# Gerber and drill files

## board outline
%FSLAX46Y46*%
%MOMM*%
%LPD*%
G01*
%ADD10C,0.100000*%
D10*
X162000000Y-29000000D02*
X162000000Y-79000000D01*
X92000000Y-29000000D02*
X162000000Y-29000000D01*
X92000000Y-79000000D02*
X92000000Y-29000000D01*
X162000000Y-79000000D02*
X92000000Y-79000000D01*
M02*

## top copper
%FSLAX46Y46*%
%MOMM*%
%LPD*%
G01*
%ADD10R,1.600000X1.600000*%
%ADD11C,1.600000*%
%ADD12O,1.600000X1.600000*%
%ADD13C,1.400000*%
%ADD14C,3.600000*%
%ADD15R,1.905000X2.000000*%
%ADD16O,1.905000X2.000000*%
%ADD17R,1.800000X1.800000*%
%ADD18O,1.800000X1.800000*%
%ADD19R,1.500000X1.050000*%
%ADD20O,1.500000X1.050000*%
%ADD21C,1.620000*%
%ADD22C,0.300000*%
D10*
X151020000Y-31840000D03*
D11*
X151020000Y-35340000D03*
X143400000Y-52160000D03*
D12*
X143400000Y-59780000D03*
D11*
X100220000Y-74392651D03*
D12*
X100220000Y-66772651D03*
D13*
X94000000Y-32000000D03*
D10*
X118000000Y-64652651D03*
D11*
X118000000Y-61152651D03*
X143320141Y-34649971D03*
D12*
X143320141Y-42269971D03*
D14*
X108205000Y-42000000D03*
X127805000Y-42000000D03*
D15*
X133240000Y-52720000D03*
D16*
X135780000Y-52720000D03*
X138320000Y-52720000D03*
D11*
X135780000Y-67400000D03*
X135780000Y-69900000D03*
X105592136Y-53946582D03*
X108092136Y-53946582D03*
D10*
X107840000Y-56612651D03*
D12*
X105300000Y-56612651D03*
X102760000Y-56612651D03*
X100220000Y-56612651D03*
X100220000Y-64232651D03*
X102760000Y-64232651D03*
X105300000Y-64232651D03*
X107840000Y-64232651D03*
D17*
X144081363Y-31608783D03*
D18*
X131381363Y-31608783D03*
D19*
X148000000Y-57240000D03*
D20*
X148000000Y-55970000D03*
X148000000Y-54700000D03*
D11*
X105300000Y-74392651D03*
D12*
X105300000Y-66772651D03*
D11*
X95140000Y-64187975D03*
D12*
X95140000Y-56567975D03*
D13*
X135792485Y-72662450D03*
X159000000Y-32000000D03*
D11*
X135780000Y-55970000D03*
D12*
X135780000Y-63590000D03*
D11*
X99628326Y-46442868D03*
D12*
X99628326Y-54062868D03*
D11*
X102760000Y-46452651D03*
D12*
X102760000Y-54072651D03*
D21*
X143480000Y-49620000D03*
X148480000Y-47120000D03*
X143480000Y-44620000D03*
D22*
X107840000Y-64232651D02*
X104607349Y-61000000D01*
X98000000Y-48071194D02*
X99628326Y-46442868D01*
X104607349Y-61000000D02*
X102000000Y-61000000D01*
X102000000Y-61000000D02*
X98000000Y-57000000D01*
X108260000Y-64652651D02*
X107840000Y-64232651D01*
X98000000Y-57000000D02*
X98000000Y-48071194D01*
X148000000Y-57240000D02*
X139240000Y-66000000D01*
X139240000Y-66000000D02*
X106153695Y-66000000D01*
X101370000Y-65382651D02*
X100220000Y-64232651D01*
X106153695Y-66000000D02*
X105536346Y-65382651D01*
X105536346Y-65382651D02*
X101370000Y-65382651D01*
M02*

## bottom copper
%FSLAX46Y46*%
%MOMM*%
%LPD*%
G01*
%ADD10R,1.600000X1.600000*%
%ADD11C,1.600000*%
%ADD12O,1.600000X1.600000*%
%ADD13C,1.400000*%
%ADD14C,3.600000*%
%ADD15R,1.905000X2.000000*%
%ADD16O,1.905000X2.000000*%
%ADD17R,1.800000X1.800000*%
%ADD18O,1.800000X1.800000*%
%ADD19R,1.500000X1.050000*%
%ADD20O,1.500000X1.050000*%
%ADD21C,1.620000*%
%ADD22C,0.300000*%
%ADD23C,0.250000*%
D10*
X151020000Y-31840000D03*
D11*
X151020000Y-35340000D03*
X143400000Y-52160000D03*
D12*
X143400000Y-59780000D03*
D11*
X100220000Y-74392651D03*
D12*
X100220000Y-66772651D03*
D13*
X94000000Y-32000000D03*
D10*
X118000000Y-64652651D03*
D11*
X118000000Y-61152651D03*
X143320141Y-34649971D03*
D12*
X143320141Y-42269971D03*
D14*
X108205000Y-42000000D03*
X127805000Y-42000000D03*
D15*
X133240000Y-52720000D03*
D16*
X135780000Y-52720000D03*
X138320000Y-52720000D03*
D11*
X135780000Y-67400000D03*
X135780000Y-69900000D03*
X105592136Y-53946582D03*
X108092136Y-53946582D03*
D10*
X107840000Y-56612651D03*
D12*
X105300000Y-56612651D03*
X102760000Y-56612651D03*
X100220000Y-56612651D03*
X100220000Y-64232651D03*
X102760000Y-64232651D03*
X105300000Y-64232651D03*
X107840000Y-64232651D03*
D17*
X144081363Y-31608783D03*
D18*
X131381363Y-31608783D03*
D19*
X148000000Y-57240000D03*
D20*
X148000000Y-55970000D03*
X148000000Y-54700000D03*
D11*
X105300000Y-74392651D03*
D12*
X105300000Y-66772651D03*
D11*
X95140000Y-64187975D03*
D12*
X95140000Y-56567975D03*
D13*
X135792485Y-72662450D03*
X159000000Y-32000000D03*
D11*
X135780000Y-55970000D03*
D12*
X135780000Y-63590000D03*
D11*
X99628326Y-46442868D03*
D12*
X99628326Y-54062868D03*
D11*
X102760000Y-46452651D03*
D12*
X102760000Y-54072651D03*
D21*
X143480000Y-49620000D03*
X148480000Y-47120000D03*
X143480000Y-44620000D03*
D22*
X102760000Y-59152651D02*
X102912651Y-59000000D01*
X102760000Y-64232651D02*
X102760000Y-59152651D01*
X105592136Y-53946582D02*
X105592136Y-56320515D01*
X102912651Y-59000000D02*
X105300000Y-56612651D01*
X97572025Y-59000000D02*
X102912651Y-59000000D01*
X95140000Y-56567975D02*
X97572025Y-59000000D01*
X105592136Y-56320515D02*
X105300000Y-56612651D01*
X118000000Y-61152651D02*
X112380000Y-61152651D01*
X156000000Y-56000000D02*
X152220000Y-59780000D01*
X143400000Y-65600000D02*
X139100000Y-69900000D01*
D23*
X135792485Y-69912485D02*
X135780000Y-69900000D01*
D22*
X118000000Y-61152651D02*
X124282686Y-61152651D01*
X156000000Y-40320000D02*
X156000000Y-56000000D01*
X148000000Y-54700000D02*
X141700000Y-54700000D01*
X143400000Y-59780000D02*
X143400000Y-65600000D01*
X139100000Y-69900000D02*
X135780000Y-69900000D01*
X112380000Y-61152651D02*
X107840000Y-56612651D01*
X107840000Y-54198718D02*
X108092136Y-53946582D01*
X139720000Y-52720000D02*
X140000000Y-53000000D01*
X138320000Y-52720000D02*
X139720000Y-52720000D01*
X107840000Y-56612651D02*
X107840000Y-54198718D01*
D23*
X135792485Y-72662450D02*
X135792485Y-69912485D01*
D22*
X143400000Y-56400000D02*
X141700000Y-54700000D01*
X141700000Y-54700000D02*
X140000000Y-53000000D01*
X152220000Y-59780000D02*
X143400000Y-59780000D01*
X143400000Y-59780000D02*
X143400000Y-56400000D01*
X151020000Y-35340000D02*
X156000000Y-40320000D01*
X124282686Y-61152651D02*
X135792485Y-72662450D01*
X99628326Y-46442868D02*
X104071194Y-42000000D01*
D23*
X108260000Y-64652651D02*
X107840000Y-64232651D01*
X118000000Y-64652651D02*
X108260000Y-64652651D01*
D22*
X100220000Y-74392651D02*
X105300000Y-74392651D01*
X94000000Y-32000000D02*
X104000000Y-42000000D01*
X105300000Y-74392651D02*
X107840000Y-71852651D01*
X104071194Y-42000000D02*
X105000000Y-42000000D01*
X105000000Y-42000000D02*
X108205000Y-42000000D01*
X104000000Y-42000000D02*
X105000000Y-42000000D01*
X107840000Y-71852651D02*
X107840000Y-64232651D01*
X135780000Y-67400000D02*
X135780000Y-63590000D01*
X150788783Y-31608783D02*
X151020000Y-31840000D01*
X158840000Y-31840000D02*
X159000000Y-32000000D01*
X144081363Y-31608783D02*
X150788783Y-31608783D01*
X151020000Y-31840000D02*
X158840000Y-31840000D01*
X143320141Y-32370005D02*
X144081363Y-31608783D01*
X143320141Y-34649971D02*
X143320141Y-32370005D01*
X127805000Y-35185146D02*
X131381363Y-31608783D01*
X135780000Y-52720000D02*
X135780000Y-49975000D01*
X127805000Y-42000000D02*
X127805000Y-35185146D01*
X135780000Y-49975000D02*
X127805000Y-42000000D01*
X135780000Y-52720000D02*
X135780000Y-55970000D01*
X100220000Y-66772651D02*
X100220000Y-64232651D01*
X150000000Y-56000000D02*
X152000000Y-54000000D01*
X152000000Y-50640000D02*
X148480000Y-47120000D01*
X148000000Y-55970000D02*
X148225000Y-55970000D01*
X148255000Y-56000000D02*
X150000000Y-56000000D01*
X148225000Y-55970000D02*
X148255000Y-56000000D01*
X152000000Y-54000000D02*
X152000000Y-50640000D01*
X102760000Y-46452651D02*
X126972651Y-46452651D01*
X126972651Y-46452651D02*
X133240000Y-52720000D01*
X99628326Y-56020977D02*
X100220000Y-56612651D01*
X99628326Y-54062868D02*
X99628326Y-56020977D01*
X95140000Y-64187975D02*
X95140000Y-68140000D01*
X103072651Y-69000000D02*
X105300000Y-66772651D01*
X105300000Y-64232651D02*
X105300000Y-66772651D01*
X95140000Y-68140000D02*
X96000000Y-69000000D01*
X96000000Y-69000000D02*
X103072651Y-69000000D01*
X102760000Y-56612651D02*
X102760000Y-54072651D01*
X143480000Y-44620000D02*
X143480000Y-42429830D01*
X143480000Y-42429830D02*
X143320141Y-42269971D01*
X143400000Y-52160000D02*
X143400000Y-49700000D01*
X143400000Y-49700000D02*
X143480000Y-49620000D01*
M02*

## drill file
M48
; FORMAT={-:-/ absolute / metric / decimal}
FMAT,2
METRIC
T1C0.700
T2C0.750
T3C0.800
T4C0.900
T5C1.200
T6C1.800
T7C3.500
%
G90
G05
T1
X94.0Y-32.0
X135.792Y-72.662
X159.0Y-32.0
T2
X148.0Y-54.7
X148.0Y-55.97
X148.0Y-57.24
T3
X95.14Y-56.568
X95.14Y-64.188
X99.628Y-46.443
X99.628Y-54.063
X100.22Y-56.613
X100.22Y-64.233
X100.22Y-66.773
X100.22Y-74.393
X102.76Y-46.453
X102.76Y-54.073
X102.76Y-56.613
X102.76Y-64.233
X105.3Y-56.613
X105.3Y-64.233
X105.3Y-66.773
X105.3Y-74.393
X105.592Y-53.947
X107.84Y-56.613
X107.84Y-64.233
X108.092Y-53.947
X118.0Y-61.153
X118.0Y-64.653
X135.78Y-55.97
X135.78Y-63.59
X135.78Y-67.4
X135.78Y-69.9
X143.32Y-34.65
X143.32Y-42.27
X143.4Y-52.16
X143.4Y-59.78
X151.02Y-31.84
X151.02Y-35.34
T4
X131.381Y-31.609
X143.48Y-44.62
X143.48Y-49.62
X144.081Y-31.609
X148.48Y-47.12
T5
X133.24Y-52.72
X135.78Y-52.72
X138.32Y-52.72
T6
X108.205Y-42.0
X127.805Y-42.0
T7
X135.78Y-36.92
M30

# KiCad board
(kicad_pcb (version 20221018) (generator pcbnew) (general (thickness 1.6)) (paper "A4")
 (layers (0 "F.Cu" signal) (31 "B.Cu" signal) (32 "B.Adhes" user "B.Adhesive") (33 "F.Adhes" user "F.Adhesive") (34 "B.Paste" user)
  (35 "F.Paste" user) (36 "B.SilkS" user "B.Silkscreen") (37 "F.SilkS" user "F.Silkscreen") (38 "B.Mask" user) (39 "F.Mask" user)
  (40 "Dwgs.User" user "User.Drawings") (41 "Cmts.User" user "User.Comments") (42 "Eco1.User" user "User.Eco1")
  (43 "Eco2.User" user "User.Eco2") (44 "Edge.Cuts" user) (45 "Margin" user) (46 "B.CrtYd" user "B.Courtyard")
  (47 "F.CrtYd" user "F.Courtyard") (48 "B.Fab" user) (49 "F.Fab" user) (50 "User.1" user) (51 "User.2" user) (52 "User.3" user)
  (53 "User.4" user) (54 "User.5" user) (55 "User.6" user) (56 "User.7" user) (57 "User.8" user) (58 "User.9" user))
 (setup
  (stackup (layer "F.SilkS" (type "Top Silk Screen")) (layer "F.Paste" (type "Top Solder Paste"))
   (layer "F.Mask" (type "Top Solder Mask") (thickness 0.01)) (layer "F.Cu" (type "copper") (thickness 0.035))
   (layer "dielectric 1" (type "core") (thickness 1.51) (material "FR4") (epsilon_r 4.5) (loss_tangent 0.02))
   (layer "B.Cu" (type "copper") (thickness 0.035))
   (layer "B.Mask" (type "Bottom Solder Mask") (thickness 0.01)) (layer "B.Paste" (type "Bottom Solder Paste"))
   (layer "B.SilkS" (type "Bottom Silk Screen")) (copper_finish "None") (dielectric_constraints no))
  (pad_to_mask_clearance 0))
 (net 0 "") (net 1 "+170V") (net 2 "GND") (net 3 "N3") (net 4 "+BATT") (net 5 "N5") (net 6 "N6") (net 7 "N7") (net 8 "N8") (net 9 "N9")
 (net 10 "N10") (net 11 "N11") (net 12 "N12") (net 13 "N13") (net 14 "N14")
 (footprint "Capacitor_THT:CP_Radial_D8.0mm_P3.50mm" (layer "F.Cu") (at 151.02 31.84 -90)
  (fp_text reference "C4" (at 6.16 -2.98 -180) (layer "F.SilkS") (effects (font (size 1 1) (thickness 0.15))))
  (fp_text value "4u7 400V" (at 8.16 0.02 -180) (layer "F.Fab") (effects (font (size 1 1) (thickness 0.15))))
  (pad "1" thru_hole rect (at 0 0 270) (size 1.6 1.6) (drill 0.8) (layers "*.Cu" "*.Mask") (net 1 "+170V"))
  (pad "2" thru_hole circle (at 3.5 0 270) (size 1.6 1.6) (drill 0.8) (layers "*.Cu" "*.Mask") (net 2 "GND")))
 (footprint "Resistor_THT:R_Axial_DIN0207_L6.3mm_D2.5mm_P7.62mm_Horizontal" (layer "F.Cu") (at 143.4 52.16 -90)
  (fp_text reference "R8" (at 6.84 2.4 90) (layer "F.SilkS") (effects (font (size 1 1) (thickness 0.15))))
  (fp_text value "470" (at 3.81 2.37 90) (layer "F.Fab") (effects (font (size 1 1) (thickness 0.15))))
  (pad "1" thru_hole circle (at 0 0 270) (size 1.6 1.6) (drill 0.8) (layers "*.Cu" "*.Mask") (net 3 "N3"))
  (pad "2" thru_hole oval (at 7.62 0 270) (size 1.6 1.6) (drill 0.8) (layers "*.Cu" "*.Mask") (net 2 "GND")))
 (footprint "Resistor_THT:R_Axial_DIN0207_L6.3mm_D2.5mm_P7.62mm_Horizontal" (layer "F.Cu") (at 100.22 74.392651 90)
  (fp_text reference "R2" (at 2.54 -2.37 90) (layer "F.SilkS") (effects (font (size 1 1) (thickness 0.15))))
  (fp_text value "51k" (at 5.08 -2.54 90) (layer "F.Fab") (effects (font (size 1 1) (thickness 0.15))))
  (pad "1" thru_hole circle (at 0 0 90) (size 1.6 1.6) (drill 0.8) (layers "*.Cu" "*.Mask") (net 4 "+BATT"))
  (pad "2" thru_hole oval (at 7.62 0 90) (size 1.6 1.6) (drill 0.8) (layers "*.Cu" "*.Mask") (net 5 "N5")))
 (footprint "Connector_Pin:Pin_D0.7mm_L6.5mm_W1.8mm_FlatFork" (layer "F.Cu") (at 94 32)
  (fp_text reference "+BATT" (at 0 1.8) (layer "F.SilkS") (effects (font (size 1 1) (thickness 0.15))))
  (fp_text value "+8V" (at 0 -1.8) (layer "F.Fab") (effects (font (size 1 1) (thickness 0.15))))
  (pad "1" thru_hole circle (at 0 0) (size 1.4 1.4) (drill 0.7) (layers "*.Cu" "*.Mask") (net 4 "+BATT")))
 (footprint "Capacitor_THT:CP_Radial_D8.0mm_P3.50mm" (layer "F.Cu") (at 118 64.652651 90)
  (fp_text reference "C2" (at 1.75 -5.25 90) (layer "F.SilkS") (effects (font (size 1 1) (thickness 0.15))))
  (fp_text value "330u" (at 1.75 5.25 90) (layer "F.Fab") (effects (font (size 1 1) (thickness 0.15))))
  (pad "1" thru_hole rect (at 0 0 90) (size 1.6 1.6) (drill 0.8) (layers "*.Cu" "*.Mask") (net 4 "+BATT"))
  (pad "2" thru_hole circle (at 3.5 0 90) (size 1.6 1.6) (drill 0.8) (layers "*.Cu" "*.Mask") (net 2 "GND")))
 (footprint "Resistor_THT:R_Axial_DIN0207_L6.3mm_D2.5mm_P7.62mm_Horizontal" (layer "F.Cu") (at 143.320141 34.649971 -90)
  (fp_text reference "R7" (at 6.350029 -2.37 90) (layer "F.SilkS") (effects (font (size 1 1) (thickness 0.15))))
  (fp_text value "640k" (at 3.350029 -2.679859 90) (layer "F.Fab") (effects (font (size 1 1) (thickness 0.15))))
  (pad "1" thru_hole circle (at 0 0 270) (size 1.6 1.6) (drill 0.8) (layers "*.Cu" "*.Mask") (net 1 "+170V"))
  (pad "2" thru_hole oval (at 7.62 0 270) (size 1.6 1.6) (drill 0.8) (layers "*.Cu" "*.Mask") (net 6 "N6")))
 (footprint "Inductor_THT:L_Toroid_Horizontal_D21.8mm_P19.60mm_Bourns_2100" (layer "F.Cu") (at 108.205 42)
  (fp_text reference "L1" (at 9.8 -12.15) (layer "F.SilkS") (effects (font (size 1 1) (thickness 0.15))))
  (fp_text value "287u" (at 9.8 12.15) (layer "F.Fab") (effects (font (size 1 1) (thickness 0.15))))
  (pad "1" thru_hole circle (at 0 0) (size 3.6 3.6) (drill 1.8) (layers "*.Cu" "*.Mask") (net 4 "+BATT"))
  (pad "2" thru_hole circle (at 19.6 0) (size 3.6 3.6) (drill 1.8) (layers "*.Cu" "*.Mask") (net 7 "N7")))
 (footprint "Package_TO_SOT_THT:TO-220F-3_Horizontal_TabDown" (layer "F.Cu") (at 133.24 52.72)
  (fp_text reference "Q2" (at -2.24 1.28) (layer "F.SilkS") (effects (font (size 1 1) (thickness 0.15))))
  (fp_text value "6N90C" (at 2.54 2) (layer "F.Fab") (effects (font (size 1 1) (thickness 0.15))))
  (pad "" np_thru_hole oval (at 2.54 -15.8) (size 3.5 3.5) (drill 3.5) (layers "*.Cu" "*.Mask"))
  (pad "1" thru_hole rect (at 0 0) (size 1.905 2) (drill 1.2) (layers "*.Cu" "*.Mask") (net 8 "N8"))
  (pad "2" thru_hole oval (at 2.54 0) (size 1.905 2) (drill 1.2) (layers "*.Cu" "*.Mask") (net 7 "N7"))
  (pad "3" thru_hole oval (at 5.08 0) (size 1.905 2) (drill 1.2) (layers "*.Cu" "*.Mask") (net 2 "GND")))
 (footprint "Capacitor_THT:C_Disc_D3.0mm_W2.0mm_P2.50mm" (layer "F.Cu") (at 135.78 67.4 -90)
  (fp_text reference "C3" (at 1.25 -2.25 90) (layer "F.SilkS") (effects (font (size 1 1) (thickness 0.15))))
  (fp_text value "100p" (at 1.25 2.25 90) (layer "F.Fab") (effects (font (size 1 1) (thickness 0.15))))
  (pad "1" thru_hole circle (at 0 0 270) (size 1.6 1.6) (drill 0.8) (layers "*.Cu" "*.Mask") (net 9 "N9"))
  (pad "2" thru_hole circle (at 2.5 0 270) (size 1.6 1.6) (drill 0.8) (layers "*.Cu" "*.Mask") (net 2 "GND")))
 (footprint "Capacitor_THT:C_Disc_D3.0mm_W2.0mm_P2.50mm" (layer "F.Cu") (at 105.592136 53.946582)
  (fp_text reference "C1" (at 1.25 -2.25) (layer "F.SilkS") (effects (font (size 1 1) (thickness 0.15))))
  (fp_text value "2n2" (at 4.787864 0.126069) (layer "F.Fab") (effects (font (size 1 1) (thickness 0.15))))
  (pad "1" thru_hole circle (at 0 0) (size 1.6 1.6) (drill 0.8) (layers "*.Cu" "*.Mask") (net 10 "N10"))
  (pad "2" thru_hole circle (at 2.5 0) (size 1.6 1.6) (drill 0.8) (layers "*.Cu" "*.Mask") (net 2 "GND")))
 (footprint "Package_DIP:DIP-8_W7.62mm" (layer "F.Cu") (at 107.84 56.612651 -90)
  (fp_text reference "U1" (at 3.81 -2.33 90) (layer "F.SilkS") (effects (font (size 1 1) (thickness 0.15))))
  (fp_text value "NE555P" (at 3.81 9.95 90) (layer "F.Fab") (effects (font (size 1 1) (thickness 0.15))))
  (pad "1" thru_hole rect (at 0 0 270) (size 1.6 1.6) (drill 0.8) (layers "*.Cu" "*.Mask") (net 2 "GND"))
  (pad "2" thru_hole oval (at 0 2.54 270) (size 1.6 1.6) (drill 0.8) (layers "*.Cu" "*.Mask") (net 10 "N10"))
  (pad "3" thru_hole oval (at 0 5.08 270) (size 1.6 1.6) (drill 0.8) (layers "*.Cu" "*.Mask") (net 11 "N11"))
  (pad "4" thru_hole oval (at 0 7.62 270) (size 1.6 1.6) (drill 0.8) (layers "*.Cu" "*.Mask") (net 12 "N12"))
  (pad "5" thru_hole oval (at 7.62 7.62 270) (size 1.6 1.6) (drill 0.8) (layers "*.Cu" "*.Mask") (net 5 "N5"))
  (pad "6" thru_hole oval (at 7.62 5.08 270) (size 1.6 1.6) (drill 0.8) (layers "*.Cu" "*.Mask") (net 10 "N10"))
  (pad "7" thru_hole oval (at 7.62 2.54 270) (size 1.6 1.6) (drill 0.8) (layers "*.Cu" "*.Mask") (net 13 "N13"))
  (pad "8" thru_hole oval (at 7.62 0 270) (size 1.6 1.6) (drill 0.8) (layers "*.Cu" "*.Mask") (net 4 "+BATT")))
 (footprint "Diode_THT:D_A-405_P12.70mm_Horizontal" (layer "F.Cu") (at 144.081363 31.608783 180)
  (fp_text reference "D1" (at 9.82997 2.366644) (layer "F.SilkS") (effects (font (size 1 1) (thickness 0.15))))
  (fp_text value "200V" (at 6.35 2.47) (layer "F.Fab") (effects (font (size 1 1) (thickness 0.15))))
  (pad "1" thru_hole rect (at 0 0 180) (size 1.8 1.8) (drill 0.9) (layers "*.Cu" "*.Mask") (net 1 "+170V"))
  (pad "2" thru_hole oval (at 12.7 0 180) (size 1.8 1.8) (drill 0.9) (layers "*.Cu" "*.Mask") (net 7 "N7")))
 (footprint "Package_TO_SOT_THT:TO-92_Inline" (layer "F.Cu") (at 148 57.24 90)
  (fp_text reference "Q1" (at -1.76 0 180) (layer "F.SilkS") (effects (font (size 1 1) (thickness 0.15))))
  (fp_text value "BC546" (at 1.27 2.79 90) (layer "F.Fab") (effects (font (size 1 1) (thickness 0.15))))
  (pad "1" thru_hole rect (at 0 0 90) (size 1.05 1.5) (drill 0.75) (layers "*.Cu" "*.Mask") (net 5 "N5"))
  (pad "2" thru_hole oval (at 1.27 0 90) (size 1.05 1.5) (drill 0.75) (layers "*.Cu" "*.Mask") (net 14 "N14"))
  (pad "3" thru_hole oval (at 2.54 0 90) (size 1.05 1.5) (drill 0.75) (layers "*.Cu" "*.Mask") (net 2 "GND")))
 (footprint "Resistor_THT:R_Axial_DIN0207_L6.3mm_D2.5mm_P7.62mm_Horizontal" (layer "F.Cu") (at 105.3 74.392651 90)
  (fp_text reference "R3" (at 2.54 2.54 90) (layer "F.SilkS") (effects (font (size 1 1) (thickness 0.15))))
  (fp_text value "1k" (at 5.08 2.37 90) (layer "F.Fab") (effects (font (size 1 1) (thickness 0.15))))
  (pad "1" thru_hole circle (at 0 0 90) (size 1.6 1.6) (drill 0.8) (layers "*.Cu" "*.Mask") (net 4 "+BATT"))
  (pad "2" thru_hole oval (at 7.62 0 90) (size 1.6 1.6) (drill 0.8) (layers "*.Cu" "*.Mask") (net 13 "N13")))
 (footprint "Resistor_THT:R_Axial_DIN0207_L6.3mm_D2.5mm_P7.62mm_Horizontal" (layer "F.Cu") (at 95.14 64.187975 90)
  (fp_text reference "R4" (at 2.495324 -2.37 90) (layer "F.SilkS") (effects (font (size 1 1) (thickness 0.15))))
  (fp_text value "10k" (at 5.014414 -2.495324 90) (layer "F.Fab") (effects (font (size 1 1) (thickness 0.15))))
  (pad "1" thru_hole circle (at 0 0 90) (size 1.6 1.6) (drill 0.8) (layers "*.Cu" "*.Mask") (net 13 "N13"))
  (pad "2" thru_hole oval (at 7.62 0 90) (size 1.6 1.6) (drill 0.8) (layers "*.Cu" "*.Mask") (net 10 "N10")))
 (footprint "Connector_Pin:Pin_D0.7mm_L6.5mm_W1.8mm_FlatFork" (layer "F.Cu") (at 135.792485 72.66245)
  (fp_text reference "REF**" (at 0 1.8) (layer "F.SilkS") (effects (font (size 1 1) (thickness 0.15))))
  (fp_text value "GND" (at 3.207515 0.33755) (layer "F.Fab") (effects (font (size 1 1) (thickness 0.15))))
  (pad "1" thru_hole circle (at 0 0) (size 1.4 1.4) (drill 0.7) (layers "*.Cu" "*.Mask") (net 2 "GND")))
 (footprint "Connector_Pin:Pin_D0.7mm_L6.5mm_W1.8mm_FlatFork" (layer "F.Cu") (at 159 32)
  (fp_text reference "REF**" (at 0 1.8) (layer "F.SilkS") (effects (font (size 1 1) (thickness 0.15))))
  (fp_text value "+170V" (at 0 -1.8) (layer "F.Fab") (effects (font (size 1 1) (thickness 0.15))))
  (pad "1" thru_hole circle (at 0 0) (size 1.4 1.4) (drill 0.7) (layers "*.Cu" "*.Mask") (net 1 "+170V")))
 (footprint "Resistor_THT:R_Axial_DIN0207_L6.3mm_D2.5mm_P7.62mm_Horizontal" (layer "F.Cu") (at 135.78 55.97 -90)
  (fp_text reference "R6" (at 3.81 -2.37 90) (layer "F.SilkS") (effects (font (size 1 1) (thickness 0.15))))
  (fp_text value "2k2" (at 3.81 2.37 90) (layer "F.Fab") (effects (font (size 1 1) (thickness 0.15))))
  (pad "1" thru_hole circle (at 0 0 270) (size 1.6 1.6) (drill 0.8) (layers "*.Cu" "*.Mask") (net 7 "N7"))
  (pad "2" thru_hole oval (at 7.62 0 270) (size 1.6 1.6) (drill 0.8) (layers "*.Cu" "*.Mask") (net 9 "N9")))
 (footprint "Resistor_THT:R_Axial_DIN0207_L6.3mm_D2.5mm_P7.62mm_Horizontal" (layer "F.Cu") (at 99.628326 46.442868 -90)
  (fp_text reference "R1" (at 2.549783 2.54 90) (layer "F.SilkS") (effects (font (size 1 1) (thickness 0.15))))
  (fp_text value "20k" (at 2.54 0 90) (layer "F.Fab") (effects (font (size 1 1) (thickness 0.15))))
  (pad "1" thru_hole circle (at 0 0 270) (size 1.6 1.6) (drill 0.8) (layers "*.Cu" "*.Mask") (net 4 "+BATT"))
  (pad "2" thru_hole oval (at 7.62 0 270) (size 1.6 1.6) (drill 0.8) (layers "*.Cu" "*.Mask") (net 12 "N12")))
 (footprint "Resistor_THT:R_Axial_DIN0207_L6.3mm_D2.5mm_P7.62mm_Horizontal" (layer "F.Cu") (at 102.76 46.452651 -90)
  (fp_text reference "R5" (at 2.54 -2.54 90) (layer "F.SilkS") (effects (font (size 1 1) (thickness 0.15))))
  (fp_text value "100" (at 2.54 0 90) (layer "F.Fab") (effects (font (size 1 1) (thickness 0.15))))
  (pad "1" thru_hole circle (at 0 0 270) (size 1.6 1.6) (drill 0.8) (layers "*.Cu" "*.Mask") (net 8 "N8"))
  (pad "2" thru_hole oval (at 7.62 0 270) (size 1.6 1.6) (drill 0.8) (layers "*.Cu" "*.Mask") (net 11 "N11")))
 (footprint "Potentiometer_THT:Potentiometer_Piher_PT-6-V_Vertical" (layer "F.Cu") (at 143.48 49.62)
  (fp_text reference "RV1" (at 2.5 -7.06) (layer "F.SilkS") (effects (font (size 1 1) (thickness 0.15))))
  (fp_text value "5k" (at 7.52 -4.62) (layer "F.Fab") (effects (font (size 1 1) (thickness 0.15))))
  (pad "1" thru_hole circle (at 0 0) (size 1.62 1.62) (drill 0.9) (layers "*.Cu" "*.Mask") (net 3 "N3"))
  (pad "2" thru_hole circle (at 5 -2.5) (size 1.62 1.62) (drill 0.9) (layers "*.Cu" "*.Mask") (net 14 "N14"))
  (pad "3" thru_hole circle (at 0 -5) (size 1.62 1.62) (drill 0.9) (layers "*.Cu" "*.Mask") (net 6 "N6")))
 (gr_line (start 162 29) (end 162 79) (stroke (width 0.1) (type default)) (layer "Edge.Cuts"))
 (gr_line (start 92 29) (end 162 29) (stroke (width 0.1) (type default)) (layer "Edge.Cuts"))
 (gr_line (start 92 79) (end 92 29) (stroke (width 0.1) (type default)) (layer "Edge.Cuts"))
 (gr_line (start 162 79) (end 92 79) (stroke (width 0.1) (type default)) (layer "Edge.Cuts"))
 (segment (start 102.76 59.152651) (end 102.912651 59) (width 0.3) (layer "B.Cu") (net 10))
 (segment (start 102.76 64.232651) (end 102.76 59.152651) (width 0.3) (layer "B.Cu") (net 10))
 (segment (start 105.592136 53.946582) (end 105.592136 56.320515) (width 0.3) (layer "B.Cu") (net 10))
 (segment (start 102.912651 59) (end 105.3 56.612651) (width 0.3) (layer "B.Cu") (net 10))
 (segment (start 97.572025 59) (end 102.912651 59) (width 0.3) (layer "B.Cu") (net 10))
 (segment (start 95.14 56.567975) (end 97.572025 59) (width 0.3) (layer "B.Cu") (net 10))
 (segment (start 105.592136 56.320515) (end 105.3 56.612651) (width 0.3) (layer "B.Cu") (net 10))
 (segment (start 118 61.152651) (end 112.38 61.152651) (width 0.3) (layer "B.Cu") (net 2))
 (segment (start 156 56) (end 152.22 59.78) (width 0.3) (layer "B.Cu") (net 2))
 (segment (start 143.4 65.6) (end 139.1 69.9) (width 0.3) (layer "B.Cu") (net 2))
 (segment (start 135.792485 69.912485) (end 135.78 69.9) (width 0.25) (layer "B.Cu") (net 2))
 (segment (start 118 61.152651) (end 124.282686 61.152651) (width 0.3) (layer "B.Cu") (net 2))
 (segment (start 156 40.32) (end 156 56) (width 0.3) (layer "B.Cu") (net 2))
 (segment (start 148 54.7) (end 141.7 54.7) (width 0.3) (layer "B.Cu") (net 2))
 (segment (start 143.4 59.78) (end 143.4 65.6) (width 0.3) (layer "B.Cu") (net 2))
 (segment (start 139.1 69.9) (end 135.78 69.9) (width 0.3) (layer "B.Cu") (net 2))
 (segment (start 112.38 61.152651) (end 107.84 56.612651) (width 0.3) (layer "B.Cu") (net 2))
 (segment (start 107.84 54.198718) (end 108.092136 53.946582) (width 0.3) (layer "B.Cu") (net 2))
 (segment (start 139.72 52.72) (end 140 53) (width 0.3) (layer "B.Cu") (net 2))
 (segment (start 138.32 52.72) (end 139.72 52.72) (width 0.3) (layer "B.Cu") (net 2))
 (segment (start 107.84 56.612651) (end 107.84 54.198718) (width 0.3) (layer "B.Cu") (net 2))
 (segment (start 135.792485 72.66245) (end 135.792485 69.912485) (width 0.25) (layer "B.Cu") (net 2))
 (segment (start 143.4 56.4) (end 141.7 54.7) (width 0.3) (layer "B.Cu") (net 2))
 (segment (start 141.7 54.7) (end 140 53) (width 0.3) (layer "B.Cu") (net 2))
 (segment (start 152.22 59.78) (end 143.4 59.78) (width 0.3) (layer "B.Cu") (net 2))
 (segment (start 143.4 59.78) (end 143.4 56.4) (width 0.3) (layer "B.Cu") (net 2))
 (segment (start 151.02 35.34) (end 156 40.32) (width 0.3) (layer "B.Cu") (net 2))
 (segment (start 124.282686 61.152651) (end 135.792485 72.66245) (width 0.3) (layer "B.Cu") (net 2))
 (segment (start 107.84 64.232651) (end 104.607349 61) (width 0.3) (layer "F.Cu") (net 4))
 (segment (start 98 48.071194) (end 99.628326 46.442868) (width 0.3) (layer "F.Cu") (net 4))
 (segment (start 104.607349 61) (end 102 61) (width 0.3) (layer "F.Cu") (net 4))
 (segment (start 102 61) (end 98 57) (width 0.3) (layer "F.Cu") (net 4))
 (segment (start 108.26 64.652651) (end 107.84 64.232651) (width 0.3) (layer "F.Cu") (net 4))
 (segment (start 98 57) (end 98 48.071194) (width 0.3) (layer "F.Cu") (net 4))
 (segment (start 99.628326 46.442868) (end 104.071194 42) (width 0.3) (layer "B.Cu") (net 4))
 (segment (start 108.26 64.652651) (end 107.84 64.232651) (width 0.25) (layer "B.Cu") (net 4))
 (segment (start 118 64.652651) (end 108.26 64.652651) (width 0.25) (layer "B.Cu") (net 4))
 (segment (start 100.22 74.392651) (end 105.3 74.392651) (width 0.3) (layer "B.Cu") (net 4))
 (segment (start 94 32) (end 104 42) (width 0.3) (layer "B.Cu") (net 4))
 (segment (start 105.3 74.392651) (end 107.84 71.852651) (width 0.3) (layer "B.Cu") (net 4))
 (segment (start 104.071194 42) (end 105 42) (width 0.3) (layer "B.Cu") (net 4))
 (segment (start 105 42) (end 108.205 42) (width 0.3) (layer "B.Cu") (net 4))
 (segment (start 104 42) (end 105 42) (width 0.3) (layer "B.Cu") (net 4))
 (segment (start 107.84 71.852651) (end 107.84 64.232651) (width 0.3) (layer "B.Cu") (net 4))
 (segment (start 135.78 67.4) (end 135.78 63.59) (width 0.3) (layer "B.Cu") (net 9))
 (segment (start 150.788783 31.608783) (end 151.02 31.84) (width 0.3) (layer "B.Cu") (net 1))
 (segment (start 158.84 31.84) (end 159 32) (width 0.3) (layer "B.Cu") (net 1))
 (segment (start 144.081363 31.608783) (end 150.788783 31.608783) (width 0.3) (layer "B.Cu") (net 1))
 (segment (start 151.02 31.84) (end 158.84 31.84) (width 0.3) (layer "B.Cu") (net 1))
 (segment (start 143.320141 32.370005) (end 144.081363 31.608783) (width 0.3) (layer "B.Cu") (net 1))
 (segment (start 143.320141 34.649971) (end 143.320141 32.370005) (width 0.3) (layer "B.Cu") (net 1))
 (segment (start 127.805 35.185146) (end 131.381363 31.608783) (width 0.3) (layer "B.Cu") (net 7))
 (segment (start 135.78 52.72) (end 135.78 49.975) (width 0.3) (layer "B.Cu") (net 7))
 (segment (start 127.805 42) (end 127.805 35.185146) (width 0.3) (layer "B.Cu") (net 7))
 (segment (start 135.78 49.975) (end 127.805 42) (width 0.3) (layer "B.Cu") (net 7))
 (segment (start 135.78 52.72) (end 135.78 55.97) (width 0.3) (layer "B.Cu") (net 7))
 (segment (start 148 57.24) (end 139.24 66) (width 0.3) (layer "F.Cu") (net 5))
 (segment (start 139.24 66) (end 106.153695 66) (width 0.3) (layer "F.Cu") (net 5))
 (segment (start 101.37 65.382651) (end 100.22 64.232651) (width 0.3) (layer "F.Cu") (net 5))
 (segment (start 106.153695 66) (end 105.536346 65.382651) (width 0.3) (layer "F.Cu") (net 5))
 (segment (start 105.536346 65.382651) (end 101.37 65.382651) (width 0.3) (layer "F.Cu") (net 5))
 (segment (start 100.22 66.772651) (end 100.22 64.232651) (width 0.3) (layer "B.Cu") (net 5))
 (segment (start 150 56) (end 152 54) (width 0.3) (layer "B.Cu") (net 14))
 (segment (start 152 50.64) (end 148.48 47.12) (width 0.3) (layer "B.Cu") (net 14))
 (segment (start 148 55.97) (end 148.225 55.97) (width 0.3) (layer "B.Cu") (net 14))
 (segment (start 148.255 56) (end 150 56) (width 0.3) (layer "B.Cu") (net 14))
 (segment (start 148.225 55.97) (end 148.255 56) (width 0.3) (layer "B.Cu") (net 14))
 (segment (start 152 54) (end 152 50.64) (width 0.3) (layer "B.Cu") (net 14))
 (segment (start 102.76 46.452651) (end 126.972651 46.452651) (width 0.3) (layer "B.Cu") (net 8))
 (segment (start 126.972651 46.452651) (end 133.24 52.72) (width 0.3) (layer "B.Cu") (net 8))
 (segment (start 99.628326 56.020977) (end 100.22 56.612651) (width 0.3) (layer "B.Cu") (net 12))
 (segment (start 99.628326 54.062868) (end 99.628326 56.020977) (width 0.3) (layer "B.Cu") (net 12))
 (segment (start 95.14 64.187975) (end 95.14 68.14) (width 0.3) (layer "B.Cu") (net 13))
 (segment (start 103.072651 69) (end 105.3 66.772651) (width 0.3) (layer "B.Cu") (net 13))
 (segment (start 105.3 64.232651) (end 105.3 66.772651) (width 0.3) (layer "B.Cu") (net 13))
 (segment (start 95.14 68.14) (end 96 69) (width 0.3) (layer "B.Cu") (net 13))
 (segment (start 96 69) (end 103.072651 69) (width 0.3) (layer "B.Cu") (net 13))
 (segment (start 102.76 56.612651) (end 102.76 54.072651) (width 0.3) (layer "B.Cu") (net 11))
 (segment (start 143.48 44.62) (end 143.48 42.42983) (width 0.3) (layer "B.Cu") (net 6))
 (segment (start 143.48 42.42983) (end 143.320141 42.269971) (width 0.3) (layer "B.Cu") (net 6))
 (segment (start 143.4 52.16) (end 143.4 49.7) (width 0.3) (layer "B.Cu") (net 3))
 (segment (start 143.4 49.7) (end 143.48 49.62) (width 0.3) (layer "B.Cu") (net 3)))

